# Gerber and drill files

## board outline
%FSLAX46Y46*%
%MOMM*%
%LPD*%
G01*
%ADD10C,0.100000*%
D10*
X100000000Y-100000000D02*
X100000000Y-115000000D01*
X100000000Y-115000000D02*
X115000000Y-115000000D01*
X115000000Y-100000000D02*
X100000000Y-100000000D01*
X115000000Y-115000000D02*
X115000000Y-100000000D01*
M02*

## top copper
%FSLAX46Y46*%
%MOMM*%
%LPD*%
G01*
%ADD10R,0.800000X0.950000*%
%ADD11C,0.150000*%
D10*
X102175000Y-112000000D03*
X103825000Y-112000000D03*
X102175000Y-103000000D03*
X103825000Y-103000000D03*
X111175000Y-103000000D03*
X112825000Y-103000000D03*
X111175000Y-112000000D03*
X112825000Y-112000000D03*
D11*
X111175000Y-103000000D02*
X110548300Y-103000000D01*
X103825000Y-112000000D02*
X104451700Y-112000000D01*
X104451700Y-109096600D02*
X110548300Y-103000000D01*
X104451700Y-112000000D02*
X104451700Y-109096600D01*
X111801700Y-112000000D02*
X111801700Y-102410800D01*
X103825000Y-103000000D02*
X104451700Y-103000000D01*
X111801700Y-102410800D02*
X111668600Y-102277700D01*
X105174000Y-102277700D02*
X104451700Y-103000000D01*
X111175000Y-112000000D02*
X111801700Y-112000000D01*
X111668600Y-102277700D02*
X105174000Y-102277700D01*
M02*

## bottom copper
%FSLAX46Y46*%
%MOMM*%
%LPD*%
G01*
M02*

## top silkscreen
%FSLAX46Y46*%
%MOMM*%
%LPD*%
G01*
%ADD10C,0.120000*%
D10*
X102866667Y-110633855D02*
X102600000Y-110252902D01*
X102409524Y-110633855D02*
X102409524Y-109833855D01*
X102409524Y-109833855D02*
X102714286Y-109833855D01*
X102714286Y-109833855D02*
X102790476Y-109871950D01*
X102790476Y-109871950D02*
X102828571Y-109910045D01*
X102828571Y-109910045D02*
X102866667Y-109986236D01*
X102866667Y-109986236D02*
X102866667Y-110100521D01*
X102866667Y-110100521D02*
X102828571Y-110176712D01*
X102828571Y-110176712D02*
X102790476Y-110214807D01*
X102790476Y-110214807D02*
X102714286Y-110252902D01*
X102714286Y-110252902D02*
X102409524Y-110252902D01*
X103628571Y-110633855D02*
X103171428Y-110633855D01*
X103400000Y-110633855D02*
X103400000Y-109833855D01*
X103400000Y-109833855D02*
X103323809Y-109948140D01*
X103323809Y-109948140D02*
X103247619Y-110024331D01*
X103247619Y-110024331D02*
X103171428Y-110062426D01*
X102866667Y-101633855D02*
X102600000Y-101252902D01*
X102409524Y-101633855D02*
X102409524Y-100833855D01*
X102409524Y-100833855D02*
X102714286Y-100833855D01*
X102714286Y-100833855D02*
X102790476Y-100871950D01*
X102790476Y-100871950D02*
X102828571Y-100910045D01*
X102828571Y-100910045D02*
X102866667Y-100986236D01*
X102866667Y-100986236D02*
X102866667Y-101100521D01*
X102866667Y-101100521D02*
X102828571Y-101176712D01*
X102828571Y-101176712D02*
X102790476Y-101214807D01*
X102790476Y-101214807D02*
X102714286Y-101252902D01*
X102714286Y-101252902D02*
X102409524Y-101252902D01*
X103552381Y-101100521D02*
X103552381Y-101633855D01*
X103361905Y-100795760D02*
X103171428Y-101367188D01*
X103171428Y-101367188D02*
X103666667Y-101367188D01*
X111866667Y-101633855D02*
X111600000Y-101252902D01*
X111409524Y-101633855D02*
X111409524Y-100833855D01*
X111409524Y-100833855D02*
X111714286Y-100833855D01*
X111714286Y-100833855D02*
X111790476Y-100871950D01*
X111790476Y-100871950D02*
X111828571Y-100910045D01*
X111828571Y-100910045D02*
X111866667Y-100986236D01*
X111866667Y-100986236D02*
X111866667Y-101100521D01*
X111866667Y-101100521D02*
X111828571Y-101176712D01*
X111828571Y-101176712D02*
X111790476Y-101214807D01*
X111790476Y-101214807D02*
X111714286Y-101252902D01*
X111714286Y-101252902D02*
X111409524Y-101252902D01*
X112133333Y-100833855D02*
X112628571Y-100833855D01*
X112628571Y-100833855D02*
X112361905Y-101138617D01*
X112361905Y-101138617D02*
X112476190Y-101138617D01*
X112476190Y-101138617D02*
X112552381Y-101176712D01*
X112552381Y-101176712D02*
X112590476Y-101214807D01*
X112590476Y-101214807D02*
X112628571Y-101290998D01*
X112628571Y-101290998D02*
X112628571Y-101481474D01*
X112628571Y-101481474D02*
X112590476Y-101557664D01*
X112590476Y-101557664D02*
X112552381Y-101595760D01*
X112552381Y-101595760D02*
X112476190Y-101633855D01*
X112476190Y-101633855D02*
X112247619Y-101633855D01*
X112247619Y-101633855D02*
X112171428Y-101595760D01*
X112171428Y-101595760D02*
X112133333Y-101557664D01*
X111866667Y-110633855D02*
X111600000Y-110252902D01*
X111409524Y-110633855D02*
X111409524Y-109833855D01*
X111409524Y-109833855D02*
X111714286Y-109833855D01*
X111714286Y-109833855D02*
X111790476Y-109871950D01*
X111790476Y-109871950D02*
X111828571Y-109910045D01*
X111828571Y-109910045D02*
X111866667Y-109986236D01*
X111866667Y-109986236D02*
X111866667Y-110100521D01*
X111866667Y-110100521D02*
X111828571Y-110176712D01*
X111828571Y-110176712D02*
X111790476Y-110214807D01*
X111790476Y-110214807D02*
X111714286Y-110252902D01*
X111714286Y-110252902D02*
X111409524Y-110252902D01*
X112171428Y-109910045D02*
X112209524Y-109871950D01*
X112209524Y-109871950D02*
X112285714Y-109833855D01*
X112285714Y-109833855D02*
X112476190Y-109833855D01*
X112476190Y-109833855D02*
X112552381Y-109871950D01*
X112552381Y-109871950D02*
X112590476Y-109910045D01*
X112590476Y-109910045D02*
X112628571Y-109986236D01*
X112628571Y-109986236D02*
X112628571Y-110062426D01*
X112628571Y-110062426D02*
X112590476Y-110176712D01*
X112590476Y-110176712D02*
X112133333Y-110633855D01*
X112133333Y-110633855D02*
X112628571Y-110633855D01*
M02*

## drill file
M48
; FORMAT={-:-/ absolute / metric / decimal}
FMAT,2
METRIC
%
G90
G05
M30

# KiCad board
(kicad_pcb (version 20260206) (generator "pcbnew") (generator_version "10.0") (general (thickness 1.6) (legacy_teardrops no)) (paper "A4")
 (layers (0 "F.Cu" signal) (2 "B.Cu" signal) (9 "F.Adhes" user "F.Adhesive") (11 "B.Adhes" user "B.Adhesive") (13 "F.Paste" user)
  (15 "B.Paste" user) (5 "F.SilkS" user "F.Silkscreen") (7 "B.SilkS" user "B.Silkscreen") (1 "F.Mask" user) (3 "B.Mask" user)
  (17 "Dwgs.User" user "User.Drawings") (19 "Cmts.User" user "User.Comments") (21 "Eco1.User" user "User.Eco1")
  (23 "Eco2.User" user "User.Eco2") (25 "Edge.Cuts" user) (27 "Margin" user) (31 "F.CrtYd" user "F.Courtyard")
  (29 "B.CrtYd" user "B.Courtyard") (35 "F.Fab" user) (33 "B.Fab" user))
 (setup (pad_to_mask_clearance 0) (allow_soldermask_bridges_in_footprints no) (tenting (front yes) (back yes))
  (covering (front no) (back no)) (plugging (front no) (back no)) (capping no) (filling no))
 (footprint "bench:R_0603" (layer "F.Cu") (at 103 112)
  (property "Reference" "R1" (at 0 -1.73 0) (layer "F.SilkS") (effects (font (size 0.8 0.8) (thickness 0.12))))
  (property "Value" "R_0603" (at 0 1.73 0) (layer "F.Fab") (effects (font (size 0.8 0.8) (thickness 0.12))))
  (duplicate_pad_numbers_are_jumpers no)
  (pad "1" smd rect (at -0.825 0) (size 0.8 0.95) (layers "F.Cu" "F.Mask" "F.Paste"))
  (pad "2" smd rect (at 0.825 0) (size 0.8 0.95) (layers "F.Cu" "F.Mask" "F.Paste") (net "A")))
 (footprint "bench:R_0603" (layer "F.Cu") (at 103 103)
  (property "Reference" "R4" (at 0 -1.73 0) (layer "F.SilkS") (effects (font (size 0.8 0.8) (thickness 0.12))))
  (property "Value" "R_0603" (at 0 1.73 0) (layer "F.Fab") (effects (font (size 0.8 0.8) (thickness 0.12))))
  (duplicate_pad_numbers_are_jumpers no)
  (pad "1" smd rect (at -0.825 0) (size 0.8 0.95) (layers "F.Cu" "F.Mask" "F.Paste"))
  (pad "2" smd rect (at 0.825 0) (size 0.8 0.95) (layers "F.Cu" "F.Mask" "F.Paste") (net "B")))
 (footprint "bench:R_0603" (layer "F.Cu") (at 112 103)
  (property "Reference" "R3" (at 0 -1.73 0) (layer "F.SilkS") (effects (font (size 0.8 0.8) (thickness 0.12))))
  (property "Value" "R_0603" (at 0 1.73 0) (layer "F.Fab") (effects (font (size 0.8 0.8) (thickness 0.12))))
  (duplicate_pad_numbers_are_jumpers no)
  (pad "1" smd rect (at -0.825 0) (size 0.8 0.95) (layers "F.Cu" "F.Mask" "F.Paste") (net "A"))
  (pad "2" smd rect (at 0.825 0) (size 0.8 0.95) (layers "F.Cu" "F.Mask" "F.Paste")))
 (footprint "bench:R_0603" (layer "F.Cu") (at 112 112)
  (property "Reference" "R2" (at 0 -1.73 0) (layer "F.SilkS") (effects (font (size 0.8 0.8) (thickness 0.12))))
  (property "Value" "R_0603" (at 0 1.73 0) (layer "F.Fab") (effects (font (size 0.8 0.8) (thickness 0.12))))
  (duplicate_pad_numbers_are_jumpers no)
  (pad "1" smd rect (at -0.825 0) (size 0.8 0.95) (layers "F.Cu" "F.Mask" "F.Paste") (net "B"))
  (pad "2" smd rect (at 0.825 0) (size 0.8 0.95) (layers "F.Cu" "F.Mask" "F.Paste")))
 (gr_line (start 100 100) (end 100 115) (stroke (width 0.1) (type solid)) (layer "Edge.Cuts"))
 (gr_line (start 100 115) (end 115 115) (stroke (width 0.1) (type solid)) (layer "Edge.Cuts"))
 (gr_line (start 115 100) (end 100 100) (stroke (width 0.1) (type solid)) (layer "Edge.Cuts"))
 (gr_line (start 115 115) (end 115 100) (stroke (width 0.1) (type solid)) (layer "Edge.Cuts"))
 (segment (start 111.175 103) (end 110.5483 103) (width 0.15) (layer "F.Cu") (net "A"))
 (segment (start 103.825 112) (end 104.4517 112) (width 0.15) (layer "F.Cu") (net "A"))
 (segment (start 104.4517 109.0966) (end 110.5483 103) (width 0.15) (layer "F.Cu") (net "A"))
 (segment (start 104.4517 112) (end 104.4517 109.0966) (width 0.15) (layer "F.Cu") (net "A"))
 (segment (start 111.8017 112) (end 111.8017 102.4108) (width 0.15) (layer "F.Cu") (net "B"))
 (segment (start 103.825 103) (end 104.4517 103) (width 0.15) (layer "F.Cu") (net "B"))
 (segment (start 111.8017 102.4108) (end 111.6686 102.2777) (width 0.15) (layer "F.Cu") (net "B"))
 (segment (start 105.174 102.2777) (end 104.4517 103) (width 0.15) (layer "F.Cu") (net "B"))
 (segment (start 111.175 112) (end 111.8017 112) (width 0.15) (layer "F.Cu") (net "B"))
 (segment (start 111.6686 102.2777) (end 105.174 102.2777) (width 0.15) (layer "F.Cu") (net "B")))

